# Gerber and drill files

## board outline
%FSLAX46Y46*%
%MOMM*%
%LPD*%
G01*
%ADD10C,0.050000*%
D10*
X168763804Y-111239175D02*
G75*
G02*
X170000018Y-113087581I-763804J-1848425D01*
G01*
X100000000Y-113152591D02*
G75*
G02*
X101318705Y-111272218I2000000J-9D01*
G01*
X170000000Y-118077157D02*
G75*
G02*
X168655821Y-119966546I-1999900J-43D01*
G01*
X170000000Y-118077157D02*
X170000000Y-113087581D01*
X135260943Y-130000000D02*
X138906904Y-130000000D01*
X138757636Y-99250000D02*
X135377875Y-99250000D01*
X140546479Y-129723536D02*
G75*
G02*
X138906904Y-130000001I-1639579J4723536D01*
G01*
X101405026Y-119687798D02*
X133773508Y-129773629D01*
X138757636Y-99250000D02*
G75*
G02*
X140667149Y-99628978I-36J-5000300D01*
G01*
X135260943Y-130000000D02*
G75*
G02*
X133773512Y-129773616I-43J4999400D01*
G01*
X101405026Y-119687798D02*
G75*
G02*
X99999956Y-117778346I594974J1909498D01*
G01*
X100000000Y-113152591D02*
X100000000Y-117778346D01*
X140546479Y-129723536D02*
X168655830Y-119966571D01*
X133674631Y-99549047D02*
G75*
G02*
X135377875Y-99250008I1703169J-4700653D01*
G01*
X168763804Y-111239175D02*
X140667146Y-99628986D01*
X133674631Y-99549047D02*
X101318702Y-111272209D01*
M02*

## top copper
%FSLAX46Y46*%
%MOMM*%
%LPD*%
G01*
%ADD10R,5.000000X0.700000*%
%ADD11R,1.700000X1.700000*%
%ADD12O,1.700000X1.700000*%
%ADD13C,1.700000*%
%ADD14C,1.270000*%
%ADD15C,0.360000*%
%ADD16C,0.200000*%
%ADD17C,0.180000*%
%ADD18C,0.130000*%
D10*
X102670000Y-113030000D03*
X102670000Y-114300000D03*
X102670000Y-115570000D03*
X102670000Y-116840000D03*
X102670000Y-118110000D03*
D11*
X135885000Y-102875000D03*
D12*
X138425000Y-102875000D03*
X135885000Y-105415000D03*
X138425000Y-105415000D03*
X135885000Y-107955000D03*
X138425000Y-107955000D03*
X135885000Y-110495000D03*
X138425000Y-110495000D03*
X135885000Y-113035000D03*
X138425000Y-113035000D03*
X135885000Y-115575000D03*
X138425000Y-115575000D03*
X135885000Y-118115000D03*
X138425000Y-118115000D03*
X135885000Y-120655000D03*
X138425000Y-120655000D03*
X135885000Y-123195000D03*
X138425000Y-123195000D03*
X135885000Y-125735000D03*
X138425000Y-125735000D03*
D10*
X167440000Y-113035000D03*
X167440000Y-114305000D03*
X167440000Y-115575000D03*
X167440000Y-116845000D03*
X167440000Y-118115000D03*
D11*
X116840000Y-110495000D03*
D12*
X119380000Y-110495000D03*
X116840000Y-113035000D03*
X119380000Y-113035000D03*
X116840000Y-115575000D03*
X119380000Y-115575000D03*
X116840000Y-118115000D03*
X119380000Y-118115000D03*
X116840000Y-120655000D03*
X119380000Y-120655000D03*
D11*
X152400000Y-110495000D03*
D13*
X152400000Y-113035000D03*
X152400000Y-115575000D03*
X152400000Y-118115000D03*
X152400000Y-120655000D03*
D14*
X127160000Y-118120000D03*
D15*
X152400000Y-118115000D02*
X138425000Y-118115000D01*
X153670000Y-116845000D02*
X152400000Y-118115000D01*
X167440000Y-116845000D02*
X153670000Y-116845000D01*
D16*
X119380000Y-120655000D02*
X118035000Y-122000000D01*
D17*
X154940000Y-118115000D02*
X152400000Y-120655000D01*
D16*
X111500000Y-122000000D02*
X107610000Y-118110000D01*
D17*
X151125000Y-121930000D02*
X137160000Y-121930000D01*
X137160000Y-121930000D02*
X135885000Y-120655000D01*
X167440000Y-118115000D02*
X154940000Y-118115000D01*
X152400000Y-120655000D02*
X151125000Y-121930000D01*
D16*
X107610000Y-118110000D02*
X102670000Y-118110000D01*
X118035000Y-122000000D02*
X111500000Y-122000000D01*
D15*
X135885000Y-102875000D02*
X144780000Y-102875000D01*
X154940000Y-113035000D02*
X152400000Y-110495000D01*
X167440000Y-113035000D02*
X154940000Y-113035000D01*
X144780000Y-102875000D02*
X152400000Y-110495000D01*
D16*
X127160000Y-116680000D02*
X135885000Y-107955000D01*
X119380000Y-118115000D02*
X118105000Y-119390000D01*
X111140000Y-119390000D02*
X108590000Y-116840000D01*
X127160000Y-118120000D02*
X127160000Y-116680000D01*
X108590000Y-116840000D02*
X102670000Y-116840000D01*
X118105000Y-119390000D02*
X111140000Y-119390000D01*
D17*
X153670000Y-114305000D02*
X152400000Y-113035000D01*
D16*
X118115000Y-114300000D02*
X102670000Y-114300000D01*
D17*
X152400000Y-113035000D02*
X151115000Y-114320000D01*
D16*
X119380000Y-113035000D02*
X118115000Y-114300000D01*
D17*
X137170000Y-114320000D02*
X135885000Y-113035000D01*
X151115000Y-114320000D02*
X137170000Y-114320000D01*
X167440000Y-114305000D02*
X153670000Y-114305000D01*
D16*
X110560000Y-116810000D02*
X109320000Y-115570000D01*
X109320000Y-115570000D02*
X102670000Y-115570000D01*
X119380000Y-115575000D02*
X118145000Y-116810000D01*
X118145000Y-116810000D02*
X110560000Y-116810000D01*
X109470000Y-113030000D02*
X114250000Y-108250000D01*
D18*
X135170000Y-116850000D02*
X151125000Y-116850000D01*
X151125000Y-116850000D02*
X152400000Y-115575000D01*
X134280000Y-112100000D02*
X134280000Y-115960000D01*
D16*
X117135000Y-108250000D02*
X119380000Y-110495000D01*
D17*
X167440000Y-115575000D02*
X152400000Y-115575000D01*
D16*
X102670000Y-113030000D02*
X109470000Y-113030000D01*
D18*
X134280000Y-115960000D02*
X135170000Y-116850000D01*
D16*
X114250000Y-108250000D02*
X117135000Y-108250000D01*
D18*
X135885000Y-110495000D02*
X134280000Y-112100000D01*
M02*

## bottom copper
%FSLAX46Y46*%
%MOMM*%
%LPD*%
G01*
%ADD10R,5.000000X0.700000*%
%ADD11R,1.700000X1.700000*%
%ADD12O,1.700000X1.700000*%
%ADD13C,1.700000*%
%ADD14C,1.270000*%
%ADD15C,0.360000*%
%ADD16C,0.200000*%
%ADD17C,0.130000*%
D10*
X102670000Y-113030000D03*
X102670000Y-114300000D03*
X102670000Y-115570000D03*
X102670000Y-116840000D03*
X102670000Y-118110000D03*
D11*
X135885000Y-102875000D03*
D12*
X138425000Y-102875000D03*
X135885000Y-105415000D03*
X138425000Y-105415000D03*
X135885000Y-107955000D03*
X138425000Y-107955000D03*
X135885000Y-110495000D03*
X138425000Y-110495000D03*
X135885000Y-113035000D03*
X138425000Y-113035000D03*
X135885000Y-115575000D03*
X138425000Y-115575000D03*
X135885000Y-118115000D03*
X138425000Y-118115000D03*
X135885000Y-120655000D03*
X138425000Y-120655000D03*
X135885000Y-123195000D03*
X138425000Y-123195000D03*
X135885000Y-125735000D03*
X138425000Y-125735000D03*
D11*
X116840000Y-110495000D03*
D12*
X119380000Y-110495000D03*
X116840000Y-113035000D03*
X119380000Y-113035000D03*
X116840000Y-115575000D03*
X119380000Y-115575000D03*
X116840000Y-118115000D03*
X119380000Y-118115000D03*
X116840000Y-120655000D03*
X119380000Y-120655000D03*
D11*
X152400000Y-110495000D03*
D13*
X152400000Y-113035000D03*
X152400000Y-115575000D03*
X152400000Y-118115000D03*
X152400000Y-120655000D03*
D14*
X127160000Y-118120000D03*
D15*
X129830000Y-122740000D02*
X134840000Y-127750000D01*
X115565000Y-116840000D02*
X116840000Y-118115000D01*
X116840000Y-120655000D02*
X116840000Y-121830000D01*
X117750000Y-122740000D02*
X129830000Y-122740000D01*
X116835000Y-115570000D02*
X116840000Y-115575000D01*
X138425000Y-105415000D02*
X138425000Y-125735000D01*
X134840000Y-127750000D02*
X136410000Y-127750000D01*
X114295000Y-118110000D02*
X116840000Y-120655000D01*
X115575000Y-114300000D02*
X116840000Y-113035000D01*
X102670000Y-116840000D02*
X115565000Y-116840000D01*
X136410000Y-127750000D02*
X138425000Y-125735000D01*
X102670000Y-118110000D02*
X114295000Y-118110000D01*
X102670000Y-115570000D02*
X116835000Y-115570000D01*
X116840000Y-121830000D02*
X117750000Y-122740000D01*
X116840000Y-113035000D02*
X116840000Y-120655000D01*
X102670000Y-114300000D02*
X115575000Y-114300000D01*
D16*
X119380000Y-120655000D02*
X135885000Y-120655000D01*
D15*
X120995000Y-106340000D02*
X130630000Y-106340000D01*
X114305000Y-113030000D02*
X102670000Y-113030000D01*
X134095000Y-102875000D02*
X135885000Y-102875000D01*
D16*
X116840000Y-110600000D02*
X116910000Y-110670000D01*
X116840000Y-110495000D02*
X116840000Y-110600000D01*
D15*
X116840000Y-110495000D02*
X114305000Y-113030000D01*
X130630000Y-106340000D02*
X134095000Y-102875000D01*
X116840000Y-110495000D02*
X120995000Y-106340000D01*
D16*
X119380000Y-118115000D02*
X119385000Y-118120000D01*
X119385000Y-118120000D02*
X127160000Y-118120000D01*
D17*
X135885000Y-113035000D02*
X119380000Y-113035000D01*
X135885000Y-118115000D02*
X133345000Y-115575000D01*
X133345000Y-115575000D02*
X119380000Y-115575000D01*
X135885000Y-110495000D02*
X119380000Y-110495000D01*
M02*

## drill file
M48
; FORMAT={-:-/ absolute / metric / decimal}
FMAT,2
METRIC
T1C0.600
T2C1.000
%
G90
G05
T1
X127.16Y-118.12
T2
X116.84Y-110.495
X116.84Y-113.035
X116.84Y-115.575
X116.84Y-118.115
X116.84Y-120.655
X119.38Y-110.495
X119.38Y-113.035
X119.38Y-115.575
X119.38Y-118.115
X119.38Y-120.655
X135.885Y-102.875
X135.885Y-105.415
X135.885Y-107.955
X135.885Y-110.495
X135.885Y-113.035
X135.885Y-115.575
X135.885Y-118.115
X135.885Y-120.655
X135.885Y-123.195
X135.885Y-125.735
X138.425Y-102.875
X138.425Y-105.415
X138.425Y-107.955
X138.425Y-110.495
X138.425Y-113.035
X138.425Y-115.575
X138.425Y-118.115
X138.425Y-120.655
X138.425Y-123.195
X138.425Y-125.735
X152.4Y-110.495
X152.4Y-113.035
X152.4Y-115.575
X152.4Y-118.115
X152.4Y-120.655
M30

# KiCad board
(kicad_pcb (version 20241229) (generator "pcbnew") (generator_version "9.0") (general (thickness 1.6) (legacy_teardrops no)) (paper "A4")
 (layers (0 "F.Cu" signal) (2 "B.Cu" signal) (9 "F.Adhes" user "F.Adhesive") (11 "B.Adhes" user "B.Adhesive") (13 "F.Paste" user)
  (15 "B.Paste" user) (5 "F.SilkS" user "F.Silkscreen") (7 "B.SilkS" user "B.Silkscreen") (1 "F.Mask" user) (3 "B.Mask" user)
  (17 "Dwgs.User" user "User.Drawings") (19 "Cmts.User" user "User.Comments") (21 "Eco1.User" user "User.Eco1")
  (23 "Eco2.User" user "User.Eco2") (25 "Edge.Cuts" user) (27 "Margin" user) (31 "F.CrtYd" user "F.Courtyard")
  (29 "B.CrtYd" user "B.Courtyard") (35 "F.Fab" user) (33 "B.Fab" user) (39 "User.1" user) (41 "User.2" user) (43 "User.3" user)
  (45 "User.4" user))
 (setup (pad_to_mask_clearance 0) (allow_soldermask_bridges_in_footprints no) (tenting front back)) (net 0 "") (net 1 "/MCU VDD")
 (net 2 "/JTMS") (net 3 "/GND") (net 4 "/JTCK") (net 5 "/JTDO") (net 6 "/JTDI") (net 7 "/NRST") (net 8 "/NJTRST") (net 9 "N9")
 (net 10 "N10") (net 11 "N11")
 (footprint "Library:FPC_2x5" (layer "F.Cu") (at 102.67 115.57 -90)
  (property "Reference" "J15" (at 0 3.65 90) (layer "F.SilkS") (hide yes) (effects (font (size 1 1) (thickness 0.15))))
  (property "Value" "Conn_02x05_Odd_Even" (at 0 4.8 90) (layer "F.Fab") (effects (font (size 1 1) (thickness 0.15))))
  (pad "1" smd rect (at -2.54 0 270) (size 0.7 5) (layers "B.Cu" "B.Mask" "B.Paste") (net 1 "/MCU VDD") (thermal_bridge_angle 45))
  (pad "2" smd rect (at -2.54 0 270) (size 0.7 5) (layers "F.Cu" "F.Mask" "F.Paste") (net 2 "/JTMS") (thermal_bridge_angle 45))
  (pad "3" smd rect (at -1.27 0 270) (size 0.7 5) (layers "B.Cu" "B.Mask" "B.Paste") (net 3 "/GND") (thermal_bridge_angle 45))
  (pad "4" smd rect (at -1.27 0 270) (size 0.7 5) (layers "F.Cu" "F.Mask" "F.Paste") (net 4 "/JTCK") (thermal_bridge_angle 45))
  (pad "5" smd rect (at 0 0 270) (size 0.7 5) (layers "B.Cu" "B.Mask" "B.Paste") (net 3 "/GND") (thermal_bridge_angle 45))
  (pad "6" smd rect (at 0 0 270) (size 0.7 5) (layers "F.Cu" "F.Mask" "F.Paste") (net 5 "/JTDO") (thermal_bridge_angle 45))
  (pad "7" smd rect (at 1.27 0 270) (size 0.7 5) (layers "B.Cu" "B.Mask" "B.Paste") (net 3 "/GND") (thermal_bridge_angle 45))
  (pad "8" smd rect (at 1.27 0 270) (size 0.7 5) (layers "F.Cu" "F.Mask" "F.Paste") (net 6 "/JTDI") (thermal_bridge_angle 45))
  (pad "9" smd rect (at 2.54 0 270) (size 0.7 5) (layers "B.Cu" "B.Mask" "B.Paste") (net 3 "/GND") (thermal_bridge_angle 45))
  (pad "10" smd rect (at 2.54 0 270) (size 0.7 5) (layers "F.Cu" "F.Mask" "F.Paste") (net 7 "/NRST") (thermal_bridge_angle 45)))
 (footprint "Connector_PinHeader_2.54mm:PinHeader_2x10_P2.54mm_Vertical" (layer "F.Cu") (at 135.885 102.875)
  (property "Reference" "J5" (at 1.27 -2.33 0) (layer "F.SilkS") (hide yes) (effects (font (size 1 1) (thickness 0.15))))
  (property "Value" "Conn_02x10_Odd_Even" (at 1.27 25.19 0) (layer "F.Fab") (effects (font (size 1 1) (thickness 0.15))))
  (pad "1" thru_hole rect (at 0 0) (size 1.7 1.7) (drill 1) (layers "*.Cu" "*.Mask") (remove_unused_layers no) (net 1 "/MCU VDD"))
  (pad "2" thru_hole oval (at 2.54 0) (size 1.7 1.7) (drill 1) (layers "*.Cu" "*.Mask") (remove_unused_layers no) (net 1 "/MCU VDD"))
  (pad "3" thru_hole oval (at 0 2.54) (size 1.7 1.7) (drill 1) (layers "*.Cu" "*.Mask") (remove_unused_layers no) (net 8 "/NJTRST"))
  (pad "4" thru_hole oval (at 2.54 2.54) (size 1.7 1.7) (drill 1) (layers "*.Cu" "*.Mask") (remove_unused_layers no) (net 3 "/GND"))
  (pad "5" thru_hole oval (at 0 5.08) (size 1.7 1.7) (drill 1) (layers "*.Cu" "*.Mask") (remove_unused_layers no) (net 6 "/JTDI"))
  (pad "6" thru_hole oval (at 2.54 5.08) (size 1.7 1.7) (drill 1) (layers "*.Cu" "*.Mask") (remove_unused_layers no) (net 3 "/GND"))
  (pad "7" thru_hole oval (at 0 7.62) (size 1.7 1.7) (drill 1) (layers "*.Cu" "*.Mask") (remove_unused_layers no) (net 2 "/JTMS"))
  (pad "8" thru_hole oval (at 2.54 7.62) (size 1.7 1.7) (drill 1) (layers "*.Cu" "*.Mask") (remove_unused_layers no) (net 3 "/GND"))
  (pad "9" thru_hole oval (at 0 10.16) (size 1.7 1.7) (drill 1) (layers "*.Cu" "*.Mask") (remove_unused_layers no) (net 4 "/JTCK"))
  (pad "10" thru_hole oval (at 2.54 10.16) (size 1.7 1.7) (drill 1) (layers "*.Cu" "*.Mask") (remove_unused_layers no) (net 3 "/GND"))
  (pad "11" thru_hole oval (at 0 12.7) (size 1.7 1.7) (drill 1) (layers "*.Cu" "*.Mask") (remove_unused_layers no) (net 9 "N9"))
  (pad "12" thru_hole oval (at 2.54 12.7) (size 1.7 1.7) (drill 1) (layers "*.Cu" "*.Mask") (remove_unused_layers no) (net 3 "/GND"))
  (pad "13" thru_hole oval (at 0 15.24) (size 1.7 1.7) (drill 1) (layers "*.Cu" "*.Mask") (remove_unused_layers no) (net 5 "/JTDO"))
  (pad "14" thru_hole oval (at 2.54 15.24) (size 1.7 1.7) (drill 1) (layers "*.Cu" "*.Mask") (remove_unused_layers no) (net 3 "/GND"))
  (pad "15" thru_hole oval (at 0 17.78) (size 1.7 1.7) (drill 1) (layers "*.Cu" "*.Mask") (remove_unused_layers no) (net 7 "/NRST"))
  (pad "16" thru_hole oval (at 2.54 17.78) (size 1.7 1.7) (drill 1) (layers "*.Cu" "*.Mask") (remove_unused_layers no) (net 3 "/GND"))
  (pad "17" thru_hole oval (at 0 20.32) (size 1.7 1.7) (drill 1) (layers "*.Cu" "*.Mask") (remove_unused_layers no) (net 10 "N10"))
  (pad "18" thru_hole oval (at 2.54 20.32) (size 1.7 1.7) (drill 1) (layers "*.Cu" "*.Mask") (remove_unused_layers no) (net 3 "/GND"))
  (pad "19" thru_hole oval (at 0 22.86) (size 1.7 1.7) (drill 1) (layers "*.Cu" "*.Mask") (remove_unused_layers no) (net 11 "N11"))
  (pad "20" thru_hole oval (at 2.54 22.86) (size 1.7 1.7) (drill 1) (layers "*.Cu" "*.Mask") (remove_unused_layers no) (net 3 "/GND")))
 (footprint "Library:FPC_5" (layer "F.Cu") (at 167.44 115.575 -90)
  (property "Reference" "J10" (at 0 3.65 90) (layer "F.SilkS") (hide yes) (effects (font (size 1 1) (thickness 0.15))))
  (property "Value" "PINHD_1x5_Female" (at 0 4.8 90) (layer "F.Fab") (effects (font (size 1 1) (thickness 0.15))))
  (pad "1" smd rect (at -2.54 0 270) (size 0.7 5) (layers "F.Cu" "F.Mask" "F.Paste") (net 1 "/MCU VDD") (thermal_bridge_angle 45))
  (pad "2" smd rect (at -1.27 0 270) (size 0.7 5) (layers "F.Cu" "F.Mask" "F.Paste") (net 4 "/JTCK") (thermal_bridge_angle 45))
  (pad "3" smd rect (at 0 0 270) (size 0.7 5) (layers "F.Cu" "F.Mask" "F.Paste") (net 2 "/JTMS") (thermal_bridge_angle 45))
  (pad "4" smd rect (at 1.27 0 270) (size 0.7 5) (layers "F.Cu" "F.Mask" "F.Paste") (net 3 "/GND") (thermal_bridge_angle 45))
  (pad "5" smd rect (at 2.54 0 270) (size 0.7 5) (layers "F.Cu" "F.Mask" "F.Paste") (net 7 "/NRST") (thermal_bridge_angle 45)))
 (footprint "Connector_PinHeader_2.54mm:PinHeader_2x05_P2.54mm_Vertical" (layer "F.Cu") (at 116.84 110.495)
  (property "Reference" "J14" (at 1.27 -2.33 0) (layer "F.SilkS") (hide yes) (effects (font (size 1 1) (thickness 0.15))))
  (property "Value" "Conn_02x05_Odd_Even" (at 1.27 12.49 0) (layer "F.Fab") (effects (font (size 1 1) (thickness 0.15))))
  (pad "1" thru_hole rect (at 0 0) (size 1.7 1.7) (drill 1) (layers "*.Cu" "*.Mask") (remove_unused_layers no) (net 1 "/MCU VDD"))
  (pad "2" thru_hole oval (at 2.54 0) (size 1.7 1.7) (drill 1) (layers "*.Cu" "*.Mask") (remove_unused_layers no) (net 2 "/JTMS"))
  (pad "3" thru_hole oval (at 0 2.54) (size 1.7 1.7) (drill 1) (layers "*.Cu" "*.Mask") (remove_unused_layers no) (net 3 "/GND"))
  (pad "4" thru_hole oval (at 2.54 2.54) (size 1.7 1.7) (drill 1) (layers "*.Cu" "*.Mask") (remove_unused_layers no) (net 4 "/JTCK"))
  (pad "5" thru_hole oval (at 0 5.08) (size 1.7 1.7) (drill 1) (layers "*.Cu" "*.Mask") (remove_unused_layers no) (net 3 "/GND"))
  (pad "6" thru_hole oval (at 2.54 5.08) (size 1.7 1.7) (drill 1) (layers "*.Cu" "*.Mask") (remove_unused_layers no) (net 5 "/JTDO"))
  (pad "7" thru_hole oval (at 0 7.62) (size 1.7 1.7) (drill 1) (layers "*.Cu" "*.Mask") (remove_unused_layers no) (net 3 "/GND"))
  (pad "8" thru_hole oval (at 2.54 7.62) (size 1.7 1.7) (drill 1) (layers "*.Cu" "*.Mask") (remove_unused_layers no) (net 6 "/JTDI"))
  (pad "9" thru_hole oval (at 0 10.16) (size 1.7 1.7) (drill 1) (layers "*.Cu" "*.Mask") (remove_unused_layers no) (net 3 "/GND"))
  (pad "10" thru_hole oval (at 2.54 10.16) (size 1.7 1.7) (drill 1) (layers "*.Cu" "*.Mask") (remove_unused_layers no) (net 7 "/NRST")))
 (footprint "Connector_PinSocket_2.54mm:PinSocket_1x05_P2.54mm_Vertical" (layer "F.Cu") (at 152.4 110.495)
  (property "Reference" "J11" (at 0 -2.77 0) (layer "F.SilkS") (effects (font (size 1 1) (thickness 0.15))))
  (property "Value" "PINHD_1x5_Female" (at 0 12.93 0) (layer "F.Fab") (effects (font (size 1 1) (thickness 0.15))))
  (pad "1" thru_hole rect (at 0 0) (size 1.7 1.7) (drill 1) (layers "*.Cu" "*.Mask") (remove_unused_layers no) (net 1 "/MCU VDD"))
  (pad "2" thru_hole circle (at 0 2.54) (size 1.7 1.7) (drill 1) (layers "*.Cu" "*.Mask") (remove_unused_layers no) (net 4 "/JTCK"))
  (pad "3" thru_hole circle (at 0 5.08) (size 1.7 1.7) (drill 1) (layers "*.Cu" "*.Mask") (remove_unused_layers no) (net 2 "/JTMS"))
  (pad "4" thru_hole circle (at 0 7.62) (size 1.7 1.7) (drill 1) (layers "*.Cu" "*.Mask") (remove_unused_layers no) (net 3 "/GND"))
  (pad "5" thru_hole circle (at 0 10.16) (size 1.7 1.7) (drill 1) (layers "*.Cu" "*.Mask") (remove_unused_layers no) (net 7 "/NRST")))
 (gr_arc (start 168.763804 111.239175) (mid 169.662469 111.975737) (end 170 113.087581) (stroke (width 0.05) (type default))
  (layer "Edge.Cuts"))
 (gr_arc (start 100 113.152591) (mid 100.362537 112.004247) (end 101.318702 111.272209) (stroke (width 0.05) (type default))
  (layer "Edge.Cuts"))
 (gr_arc (start 170 118.077157) (mid 169.629688 119.23656) (end 168.65583 119.966571) (stroke (width 0.05) (type default))
  (layer "Edge.Cuts"))
 (gr_line (start 170 118.077157) (end 170 113.087581) (stroke (width 0.05) (type default)) (layer "Edge.Cuts"))
 (gr_line (start 135.260943 130) (end 138.906904 130) (stroke (width 0.05) (type default)) (layer "Edge.Cuts"))
 (gr_line (start 138.757636 99.25) (end 135.377875 99.25) (stroke (width 0.05) (type default)) (layer "Edge.Cuts"))
 (gr_arc (start 140.546479 129.723536) (mid 139.738264 129.930399) (end 138.906904 130) (stroke (width 0.05) (type default))
  (layer "Edge.Cuts"))
 (gr_line (start 101.405026 119.687798) (end 133.773508 129.773629) (stroke (width 0.05) (type default)) (layer "Edge.Cuts"))
 (gr_arc (start 138.757636 99.25) (mid 139.731012 99.345668) (end 140.667146 99.628986) (stroke (width 0.05) (type default))
  (layer "Edge.Cuts"))
 (gr_arc (start 135.260943 130) (mid 134.508661 129.94309) (end 133.773508 129.773629) (stroke (width 0.05) (type default))
  (layer "Edge.Cuts"))
 (gr_arc (start 101.405026 119.687798) (mid 100.389108 118.963684) (end 100 117.778346) (stroke (width 0.05) (type default))
  (layer "Edge.Cuts"))
 (gr_line (start 100 113.152591) (end 100 117.778346) (stroke (width 0.05) (type default)) (layer "Edge.Cuts"))
 (gr_line (start 140.546479 129.723536) (end 168.65583 119.966571) (stroke (width 0.05) (type default)) (layer "Edge.Cuts"))
 (gr_arc (start 133.674631 99.549047) (mid 134.513226 99.325325) (end 135.377875 99.25) (stroke (width 0.05) (type default))
  (layer "Edge.Cuts"))
 (gr_line (start 168.763804 111.239175) (end 140.667146 99.628986) (stroke (width 0.05) (type default)) (layer "Edge.Cuts"))
 (gr_line (start 133.674631 99.549047) (end 101.318702 111.272209) (stroke (width 0.05) (type default)) (layer "Edge.Cuts"))
 (segment (start 152.4 118.115) (end 138.425 118.115) (width 0.36) (layer "F.Cu") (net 3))
 (segment (start 153.67 116.845) (end 152.4 118.115) (width 0.36) (layer "F.Cu") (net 3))
 (segment (start 167.44 116.845) (end 153.67 116.845) (width 0.36) (layer "F.Cu") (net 3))
 (segment (start 129.83 122.74) (end 134.84 127.75) (width 0.36) (layer "B.Cu") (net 3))
 (segment (start 115.565 116.84) (end 116.84 118.115) (width 0.36) (layer "B.Cu") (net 3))
 (segment (start 116.84 120.655) (end 116.84 121.83) (width 0.36) (layer "B.Cu") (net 3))
 (segment (start 117.75 122.74) (end 129.83 122.74) (width 0.36) (layer "B.Cu") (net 3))
 (segment (start 116.835 115.57) (end 116.84 115.575) (width 0.36) (layer "B.Cu") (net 3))
 (segment (start 138.425 105.415) (end 138.425 125.735) (width 0.36) (layer "B.Cu") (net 3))
 (segment (start 134.84 127.75) (end 136.41 127.75) (width 0.36) (layer "B.Cu") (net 3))
 (segment (start 114.295 118.11) (end 116.84 120.655) (width 0.36) (layer "B.Cu") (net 3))
 (segment (start 115.575 114.3) (end 116.84 113.035) (width 0.36) (layer "B.Cu") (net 3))
 (segment (start 102.67 116.84) (end 115.565 116.84) (width 0.36) (layer "B.Cu") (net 3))
 (segment (start 136.41 127.75) (end 138.425 125.735) (width 0.36) (layer "B.Cu") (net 3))
 (segment (start 102.67 118.11) (end 114.295 118.11) (width 0.36) (layer "B.Cu") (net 3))
 (segment (start 102.67 115.57) (end 116.835 115.57) (width 0.36) (layer "B.Cu") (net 3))
 (segment (start 116.84 121.83) (end 117.75 122.74) (width 0.36) (layer "B.Cu") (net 3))
 (segment (start 116.84 113.035) (end 116.84 120.655) (width 0.36) (layer "B.Cu") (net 3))
 (segment (start 102.67 114.3) (end 115.575 114.3) (width 0.36) (layer "B.Cu") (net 3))
 (segment (start 119.38 120.655) (end 118.035 122) (width 0.2) (layer "F.Cu") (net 7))
 (segment (start 154.94 118.115) (end 152.4 120.655) (width 0.18) (layer "F.Cu") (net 7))
 (segment (start 111.5 122) (end 107.61 118.11) (width 0.2) (layer "F.Cu") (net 7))
 (segment (start 151.125 121.93) (end 137.16 121.93) (width 0.18) (layer "F.Cu") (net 7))
 (segment (start 137.16 121.93) (end 135.885 120.655) (width 0.18) (layer "F.Cu") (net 7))
 (segment (start 167.44 118.115) (end 154.94 118.115) (width 0.18) (layer "F.Cu") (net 7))
 (segment (start 152.4 120.655) (end 151.125 121.93) (width 0.18) (layer "F.Cu") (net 7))
 (segment (start 107.61 118.11) (end 102.67 118.11) (width 0.2) (layer "F.Cu") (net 7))
 (segment (start 118.035 122) (end 111.5 122) (width 0.2) (layer "F.Cu") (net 7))
 (segment (start 119.38 120.655) (end 135.885 120.655) (width 0.2) (layer "B.Cu") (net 7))
 (segment (start 135.885 102.875) (end 144.78 102.875) (width 0.36) (layer "F.Cu") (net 1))
 (segment (start 154.94 113.035) (end 152.4 110.495) (width 0.36) (layer "F.Cu") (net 1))
 (segment (start 167.44 113.035) (end 154.94 113.035) (width 0.36) (layer "F.Cu") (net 1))
 (segment (start 144.78 102.875) (end 152.4 110.495) (width 0.36) (layer "F.Cu") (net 1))
 (segment (start 120.995 106.34) (end 130.63 106.34) (width 0.36) (layer "B.Cu") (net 1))
 (segment (start 114.305 113.03) (end 102.67 113.03) (width 0.36) (layer "B.Cu") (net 1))
 (segment (start 134.095 102.875) (end 135.885 102.875) (width 0.36) (layer "B.Cu") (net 1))
 (segment (start 116.84 110.6) (end 116.91 110.67) (width 0.2) (layer "B.Cu") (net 1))
 (segment (start 116.84 110.495) (end 116.84 110.6) (width 0.2) (layer "B.Cu") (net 1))
 (segment (start 116.84 110.495) (end 114.305 113.03) (width 0.36) (layer "B.Cu") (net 1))
 (segment (start 130.63 106.34) (end 134.095 102.875) (width 0.36) (layer "B.Cu") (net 1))
 (segment (start 116.84 110.495) (end 120.995 106.34) (width 0.36) (layer "B.Cu") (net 1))
 (segment (start 127.16 116.68) (end 135.885 107.955) (width 0.2) (layer "F.Cu") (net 6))
 (segment (start 119.38 118.115) (end 118.105 119.39) (width 0.2) (layer "F.Cu") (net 6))
 (segment (start 111.14 119.39) (end 108.59 116.84) (width 0.2) (layer "F.Cu") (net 6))
 (segment (start 127.16 118.12) (end 127.16 116.68) (width 0.2) (layer "F.Cu") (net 6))
 (segment (start 108.59 116.84) (end 102.67 116.84) (width 0.2) (layer "F.Cu") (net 6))
 (segment (start 118.105 119.39) (end 111.14 119.39) (width 0.2) (layer "F.Cu") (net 6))
 (via (at 127.16 118.12) (size 1.27) (drill 0.6) (layers "F.Cu" "B.Cu") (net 6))
 (segment (start 119.38 118.115) (end 119.385 118.12) (width 0.2) (layer "B.Cu") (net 6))
 (segment (start 119.385 118.12) (end 127.16 118.12) (width 0.2) (layer "B.Cu") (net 6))
 (segment (start 153.67 114.305) (end 152.4 113.035) (width 0.18) (layer "F.Cu") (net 4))
 (segment (start 118.115 114.3) (end 102.67 114.3) (width 0.2) (layer "F.Cu") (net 4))
 (segment (start 152.4 113.035) (end 151.115 114.32) (width 0.18) (layer "F.Cu") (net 4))
 (segment (start 119.38 113.035) (end 118.115 114.3) (width 0.2) (layer "F.Cu") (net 4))
 (segment (start 137.17 114.32) (end 135.885 113.035) (width 0.18) (layer "F.Cu") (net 4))
 (segment (start 151.115 114.32) (end 137.17 114.32) (width 0.18) (layer "F.Cu") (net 4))
 (segment (start 167.44 114.305) (end 153.67 114.305) (width 0.18) (layer "F.Cu") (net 4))
 (segment (start 135.885 113.035) (end 119.38 113.035) (width 0.13) (layer "B.Cu") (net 4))
 (segment (start 110.56 116.81) (end 109.32 115.57) (width 0.2) (layer "F.Cu") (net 5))
 (segment (start 109.32 115.57) (end 102.67 115.57) (width 0.2) (layer "F.Cu") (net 5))
 (segment (start 119.38 115.575) (end 118.145 116.81) (width 0.2) (layer "F.Cu") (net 5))
 (segment (start 118.145 116.81) (end 110.56 116.81) (width 0.2) (layer "F.Cu") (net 5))
 (segment (start 135.885 118.115) (end 133.345 115.575) (width 0.13) (layer "B.Cu") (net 5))
 (segment (start 133.345 115.575) (end 119.38 115.575) (width 0.13) (layer "B.Cu") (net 5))
 (segment (start 109.47 113.03) (end 114.25 108.25) (width 0.2) (layer "F.Cu") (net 2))
 (segment (start 135.17 116.85) (end 151.125 116.85) (width 0.13) (layer "F.Cu") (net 2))
 (segment (start 151.125 116.85) (end 152.4 115.575) (width 0.13) (layer "F.Cu") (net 2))
 (segment (start 134.28 112.1) (end 134.28 115.96) (width 0.13) (layer "F.Cu") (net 2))
 (segment (start 117.135 108.25) (end 119.38 110.495) (width 0.2) (layer "F.Cu") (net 2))
 (segment (start 167.44 115.575) (end 152.4 115.575) (width 0.18) (layer "F.Cu") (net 2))
 (segment (start 102.67 113.03) (end 109.47 113.03) (width 0.2) (layer "F.Cu") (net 2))
 (segment (start 134.28 115.96) (end 135.17 116.85) (width 0.13) (layer "F.Cu") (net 2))
 (segment (start 114.25 108.25) (end 117.135 108.25) (width 0.2) (layer "F.Cu") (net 2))
 (segment (start 135.885 110.495) (end 134.28 112.1) (width 0.13) (layer "F.Cu") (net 2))
 (segment (start 135.885 110.495) (end 119.38 110.495) (width 0.13) (layer "B.Cu") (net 2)))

